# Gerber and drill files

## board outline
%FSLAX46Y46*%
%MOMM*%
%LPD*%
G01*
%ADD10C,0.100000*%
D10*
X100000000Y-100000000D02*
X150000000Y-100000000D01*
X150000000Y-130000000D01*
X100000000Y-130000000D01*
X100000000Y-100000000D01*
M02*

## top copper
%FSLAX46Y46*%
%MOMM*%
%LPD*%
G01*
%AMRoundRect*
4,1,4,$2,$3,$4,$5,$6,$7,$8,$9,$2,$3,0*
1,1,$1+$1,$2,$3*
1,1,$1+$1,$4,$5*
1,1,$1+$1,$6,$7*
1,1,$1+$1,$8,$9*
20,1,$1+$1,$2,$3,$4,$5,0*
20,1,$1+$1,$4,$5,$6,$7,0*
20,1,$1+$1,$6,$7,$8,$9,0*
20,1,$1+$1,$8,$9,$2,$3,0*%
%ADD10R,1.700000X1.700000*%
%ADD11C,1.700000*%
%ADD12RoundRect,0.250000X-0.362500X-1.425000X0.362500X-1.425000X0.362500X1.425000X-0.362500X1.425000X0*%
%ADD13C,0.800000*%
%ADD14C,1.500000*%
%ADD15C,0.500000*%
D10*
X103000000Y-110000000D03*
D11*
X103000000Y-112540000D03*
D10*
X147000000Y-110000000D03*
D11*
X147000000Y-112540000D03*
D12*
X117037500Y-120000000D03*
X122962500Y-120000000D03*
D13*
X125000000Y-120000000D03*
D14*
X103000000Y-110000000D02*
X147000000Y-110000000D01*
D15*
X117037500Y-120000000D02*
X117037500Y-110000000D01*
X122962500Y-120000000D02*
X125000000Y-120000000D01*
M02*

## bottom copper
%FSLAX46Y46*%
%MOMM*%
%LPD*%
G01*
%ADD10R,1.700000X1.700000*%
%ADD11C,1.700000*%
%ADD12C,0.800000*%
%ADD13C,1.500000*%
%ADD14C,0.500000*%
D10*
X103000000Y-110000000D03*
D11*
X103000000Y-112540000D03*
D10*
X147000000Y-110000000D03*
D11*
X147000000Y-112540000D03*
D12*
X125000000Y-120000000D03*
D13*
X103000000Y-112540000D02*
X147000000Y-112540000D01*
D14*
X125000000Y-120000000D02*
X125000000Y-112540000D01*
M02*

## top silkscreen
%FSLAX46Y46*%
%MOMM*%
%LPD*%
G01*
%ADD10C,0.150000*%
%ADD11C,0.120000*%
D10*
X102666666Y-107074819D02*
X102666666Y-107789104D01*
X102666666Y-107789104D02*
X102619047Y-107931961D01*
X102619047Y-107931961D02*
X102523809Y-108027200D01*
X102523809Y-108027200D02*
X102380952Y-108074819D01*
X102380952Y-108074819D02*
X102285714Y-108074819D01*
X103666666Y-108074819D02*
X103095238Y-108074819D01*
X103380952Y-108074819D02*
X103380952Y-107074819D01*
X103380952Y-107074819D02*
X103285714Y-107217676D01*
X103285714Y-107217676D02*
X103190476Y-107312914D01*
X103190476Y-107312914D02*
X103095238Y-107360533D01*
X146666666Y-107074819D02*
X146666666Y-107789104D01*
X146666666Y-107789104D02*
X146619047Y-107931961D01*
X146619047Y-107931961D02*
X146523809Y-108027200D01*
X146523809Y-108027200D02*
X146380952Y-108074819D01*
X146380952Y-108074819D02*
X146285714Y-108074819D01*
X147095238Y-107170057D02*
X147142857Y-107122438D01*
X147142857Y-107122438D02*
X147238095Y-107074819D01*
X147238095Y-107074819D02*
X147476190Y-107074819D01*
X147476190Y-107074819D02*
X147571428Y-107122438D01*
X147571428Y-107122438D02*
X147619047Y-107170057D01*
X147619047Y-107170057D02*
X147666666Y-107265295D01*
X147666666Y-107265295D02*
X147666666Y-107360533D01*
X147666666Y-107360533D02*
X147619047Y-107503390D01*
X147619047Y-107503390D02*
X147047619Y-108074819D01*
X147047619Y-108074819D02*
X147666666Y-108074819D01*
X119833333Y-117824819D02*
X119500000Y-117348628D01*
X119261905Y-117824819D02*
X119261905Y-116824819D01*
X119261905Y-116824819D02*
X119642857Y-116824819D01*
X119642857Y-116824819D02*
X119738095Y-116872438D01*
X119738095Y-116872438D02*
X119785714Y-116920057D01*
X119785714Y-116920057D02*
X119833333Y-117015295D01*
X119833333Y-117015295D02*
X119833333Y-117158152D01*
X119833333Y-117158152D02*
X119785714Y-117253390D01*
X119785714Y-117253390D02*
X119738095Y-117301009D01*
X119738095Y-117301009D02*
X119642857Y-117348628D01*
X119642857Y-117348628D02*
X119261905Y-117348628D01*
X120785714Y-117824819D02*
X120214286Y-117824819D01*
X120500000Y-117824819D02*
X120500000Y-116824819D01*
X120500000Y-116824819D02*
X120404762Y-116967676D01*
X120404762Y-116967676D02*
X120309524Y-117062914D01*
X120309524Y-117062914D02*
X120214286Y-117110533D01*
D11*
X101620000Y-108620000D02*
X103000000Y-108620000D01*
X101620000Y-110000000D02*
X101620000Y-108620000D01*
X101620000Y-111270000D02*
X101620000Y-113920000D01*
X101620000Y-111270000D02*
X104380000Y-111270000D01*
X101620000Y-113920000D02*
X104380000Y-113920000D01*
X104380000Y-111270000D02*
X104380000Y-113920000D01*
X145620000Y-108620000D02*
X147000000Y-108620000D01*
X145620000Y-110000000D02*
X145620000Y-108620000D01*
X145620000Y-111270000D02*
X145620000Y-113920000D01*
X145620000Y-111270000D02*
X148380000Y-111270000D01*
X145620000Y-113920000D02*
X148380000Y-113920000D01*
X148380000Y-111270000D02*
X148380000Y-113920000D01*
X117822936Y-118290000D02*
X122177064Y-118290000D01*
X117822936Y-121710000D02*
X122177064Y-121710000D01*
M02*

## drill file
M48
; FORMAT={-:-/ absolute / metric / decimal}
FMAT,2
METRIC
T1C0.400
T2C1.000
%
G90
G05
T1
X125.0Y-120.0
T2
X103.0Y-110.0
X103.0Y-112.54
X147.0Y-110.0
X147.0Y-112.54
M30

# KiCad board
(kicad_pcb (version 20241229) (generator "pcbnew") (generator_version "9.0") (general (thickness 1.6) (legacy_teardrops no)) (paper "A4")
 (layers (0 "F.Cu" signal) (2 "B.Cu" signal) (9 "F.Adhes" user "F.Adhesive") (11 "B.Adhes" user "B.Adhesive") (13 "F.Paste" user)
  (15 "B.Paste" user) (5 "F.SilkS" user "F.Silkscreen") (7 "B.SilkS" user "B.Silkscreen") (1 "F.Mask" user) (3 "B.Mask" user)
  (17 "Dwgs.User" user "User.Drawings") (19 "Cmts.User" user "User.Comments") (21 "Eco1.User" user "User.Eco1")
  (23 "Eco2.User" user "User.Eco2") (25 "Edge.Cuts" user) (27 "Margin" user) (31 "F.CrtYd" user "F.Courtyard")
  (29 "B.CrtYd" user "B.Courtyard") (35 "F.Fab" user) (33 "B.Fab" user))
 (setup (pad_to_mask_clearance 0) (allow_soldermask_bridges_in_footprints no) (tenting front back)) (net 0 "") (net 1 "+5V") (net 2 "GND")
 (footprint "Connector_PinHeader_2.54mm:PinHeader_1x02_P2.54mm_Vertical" (layer "F.Cu") (at 103 110)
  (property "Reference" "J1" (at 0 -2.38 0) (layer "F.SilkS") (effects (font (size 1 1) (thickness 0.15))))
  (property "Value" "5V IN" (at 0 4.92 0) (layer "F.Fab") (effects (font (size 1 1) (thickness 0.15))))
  (fp_line (start -1.38 -1.38) (end 0 -1.38) (stroke (width 0.12) (type solid)) (layer "F.SilkS"))
  (fp_line (start -1.38 0) (end -1.38 -1.38) (stroke (width 0.12) (type solid)) (layer "F.SilkS"))
  (fp_line (start -1.38 1.27) (end -1.38 3.92) (stroke (width 0.12) (type solid)) (layer "F.SilkS"))
  (fp_line (start -1.38 1.27) (end 1.38 1.27) (stroke (width 0.12) (type solid)) (layer "F.SilkS"))
  (fp_line (start -1.38 3.92) (end 1.38 3.92) (stroke (width 0.12) (type solid)) (layer "F.SilkS"))
  (fp_line (start 1.38 1.27) (end 1.38 3.92) (stroke (width 0.12) (type solid)) (layer "F.SilkS"))
  (pad "1" thru_hole rect (at 0 0) (size 1.7 1.7) (drill 1) (layers "*.Cu" "*.Mask") (remove_unused_layers no) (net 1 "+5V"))
  (pad "2" thru_hole circle (at 0 2.54) (size 1.7 1.7) (drill 1) (layers "*.Cu" "*.Mask") (remove_unused_layers no) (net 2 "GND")))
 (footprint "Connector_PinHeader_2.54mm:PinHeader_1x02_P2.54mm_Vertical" (layer "F.Cu") (at 147 110)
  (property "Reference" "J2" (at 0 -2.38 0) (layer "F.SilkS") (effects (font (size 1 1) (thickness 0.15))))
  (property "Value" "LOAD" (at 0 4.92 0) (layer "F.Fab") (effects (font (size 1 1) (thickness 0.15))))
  (fp_line (start -1.38 -1.38) (end 0 -1.38) (stroke (width 0.12) (type solid)) (layer "F.SilkS"))
  (fp_line (start -1.38 0) (end -1.38 -1.38) (stroke (width 0.12) (type solid)) (layer "F.SilkS"))
  (fp_line (start -1.38 1.27) (end -1.38 3.92) (stroke (width 0.12) (type solid)) (layer "F.SilkS"))
  (fp_line (start -1.38 1.27) (end 1.38 1.27) (stroke (width 0.12) (type solid)) (layer "F.SilkS"))
  (fp_line (start -1.38 3.92) (end 1.38 3.92) (stroke (width 0.12) (type solid)) (layer "F.SilkS"))
  (fp_line (start 1.38 1.27) (end 1.38 3.92) (stroke (width 0.12) (type solid)) (layer "F.SilkS"))
  (pad "1" thru_hole rect (at 0 0) (size 1.7 1.7) (drill 1) (layers "*.Cu" "*.Mask") (remove_unused_layers no) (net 1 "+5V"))
  (pad "2" thru_hole circle (at 0 2.54) (size 1.7 1.7) (drill 1) (layers "*.Cu" "*.Mask") (remove_unused_layers no) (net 2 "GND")))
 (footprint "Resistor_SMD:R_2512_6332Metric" (layer "F.Cu") (at 120 120)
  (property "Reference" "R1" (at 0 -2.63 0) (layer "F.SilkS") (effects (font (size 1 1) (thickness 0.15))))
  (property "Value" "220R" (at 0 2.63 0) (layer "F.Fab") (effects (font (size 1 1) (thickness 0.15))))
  (fp_line (start -2.177064 -1.71) (end 2.177064 -1.71) (stroke (width 0.12) (type solid)) (layer "F.SilkS"))
  (fp_line (start -2.177064 1.71) (end 2.177064 1.71) (stroke (width 0.12) (type solid)) (layer "F.SilkS"))
  (pad "1" smd roundrect (at -2.9625 0) (size 1.225 3.35) (layers "F.Cu" "F.Mask" "F.Paste") (roundrect_rratio 0.204082) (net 1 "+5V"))
  (pad "2" smd roundrect (at 2.9625 0) (size 1.225 3.35) (layers "F.Cu" "F.Mask" "F.Paste") (roundrect_rratio 0.204082) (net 2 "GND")))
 (gr_rect (start 100 100) (end 150 130) (stroke (width 0.1) (type default)) (fill no) (layer "Edge.Cuts"))
 (segment (start 103 110) (end 147 110) (width 1.5) (layer "F.Cu") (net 1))
 (segment (start 103 112.54) (end 147 112.54) (width 1.5) (layer "B.Cu") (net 2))
 (segment (start 117.0375 120) (end 117.0375 110) (width 0.5) (layer "F.Cu") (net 1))
 (segment (start 122.9625 120) (end 125 120) (width 0.5) (layer "F.Cu") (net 2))
 (segment (start 125 120) (end 125 112.54) (width 0.5) (layer "B.Cu") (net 2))
 (via (at 125 120) (size 0.8) (drill 0.4) (layers "F.Cu" "B.Cu") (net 2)))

